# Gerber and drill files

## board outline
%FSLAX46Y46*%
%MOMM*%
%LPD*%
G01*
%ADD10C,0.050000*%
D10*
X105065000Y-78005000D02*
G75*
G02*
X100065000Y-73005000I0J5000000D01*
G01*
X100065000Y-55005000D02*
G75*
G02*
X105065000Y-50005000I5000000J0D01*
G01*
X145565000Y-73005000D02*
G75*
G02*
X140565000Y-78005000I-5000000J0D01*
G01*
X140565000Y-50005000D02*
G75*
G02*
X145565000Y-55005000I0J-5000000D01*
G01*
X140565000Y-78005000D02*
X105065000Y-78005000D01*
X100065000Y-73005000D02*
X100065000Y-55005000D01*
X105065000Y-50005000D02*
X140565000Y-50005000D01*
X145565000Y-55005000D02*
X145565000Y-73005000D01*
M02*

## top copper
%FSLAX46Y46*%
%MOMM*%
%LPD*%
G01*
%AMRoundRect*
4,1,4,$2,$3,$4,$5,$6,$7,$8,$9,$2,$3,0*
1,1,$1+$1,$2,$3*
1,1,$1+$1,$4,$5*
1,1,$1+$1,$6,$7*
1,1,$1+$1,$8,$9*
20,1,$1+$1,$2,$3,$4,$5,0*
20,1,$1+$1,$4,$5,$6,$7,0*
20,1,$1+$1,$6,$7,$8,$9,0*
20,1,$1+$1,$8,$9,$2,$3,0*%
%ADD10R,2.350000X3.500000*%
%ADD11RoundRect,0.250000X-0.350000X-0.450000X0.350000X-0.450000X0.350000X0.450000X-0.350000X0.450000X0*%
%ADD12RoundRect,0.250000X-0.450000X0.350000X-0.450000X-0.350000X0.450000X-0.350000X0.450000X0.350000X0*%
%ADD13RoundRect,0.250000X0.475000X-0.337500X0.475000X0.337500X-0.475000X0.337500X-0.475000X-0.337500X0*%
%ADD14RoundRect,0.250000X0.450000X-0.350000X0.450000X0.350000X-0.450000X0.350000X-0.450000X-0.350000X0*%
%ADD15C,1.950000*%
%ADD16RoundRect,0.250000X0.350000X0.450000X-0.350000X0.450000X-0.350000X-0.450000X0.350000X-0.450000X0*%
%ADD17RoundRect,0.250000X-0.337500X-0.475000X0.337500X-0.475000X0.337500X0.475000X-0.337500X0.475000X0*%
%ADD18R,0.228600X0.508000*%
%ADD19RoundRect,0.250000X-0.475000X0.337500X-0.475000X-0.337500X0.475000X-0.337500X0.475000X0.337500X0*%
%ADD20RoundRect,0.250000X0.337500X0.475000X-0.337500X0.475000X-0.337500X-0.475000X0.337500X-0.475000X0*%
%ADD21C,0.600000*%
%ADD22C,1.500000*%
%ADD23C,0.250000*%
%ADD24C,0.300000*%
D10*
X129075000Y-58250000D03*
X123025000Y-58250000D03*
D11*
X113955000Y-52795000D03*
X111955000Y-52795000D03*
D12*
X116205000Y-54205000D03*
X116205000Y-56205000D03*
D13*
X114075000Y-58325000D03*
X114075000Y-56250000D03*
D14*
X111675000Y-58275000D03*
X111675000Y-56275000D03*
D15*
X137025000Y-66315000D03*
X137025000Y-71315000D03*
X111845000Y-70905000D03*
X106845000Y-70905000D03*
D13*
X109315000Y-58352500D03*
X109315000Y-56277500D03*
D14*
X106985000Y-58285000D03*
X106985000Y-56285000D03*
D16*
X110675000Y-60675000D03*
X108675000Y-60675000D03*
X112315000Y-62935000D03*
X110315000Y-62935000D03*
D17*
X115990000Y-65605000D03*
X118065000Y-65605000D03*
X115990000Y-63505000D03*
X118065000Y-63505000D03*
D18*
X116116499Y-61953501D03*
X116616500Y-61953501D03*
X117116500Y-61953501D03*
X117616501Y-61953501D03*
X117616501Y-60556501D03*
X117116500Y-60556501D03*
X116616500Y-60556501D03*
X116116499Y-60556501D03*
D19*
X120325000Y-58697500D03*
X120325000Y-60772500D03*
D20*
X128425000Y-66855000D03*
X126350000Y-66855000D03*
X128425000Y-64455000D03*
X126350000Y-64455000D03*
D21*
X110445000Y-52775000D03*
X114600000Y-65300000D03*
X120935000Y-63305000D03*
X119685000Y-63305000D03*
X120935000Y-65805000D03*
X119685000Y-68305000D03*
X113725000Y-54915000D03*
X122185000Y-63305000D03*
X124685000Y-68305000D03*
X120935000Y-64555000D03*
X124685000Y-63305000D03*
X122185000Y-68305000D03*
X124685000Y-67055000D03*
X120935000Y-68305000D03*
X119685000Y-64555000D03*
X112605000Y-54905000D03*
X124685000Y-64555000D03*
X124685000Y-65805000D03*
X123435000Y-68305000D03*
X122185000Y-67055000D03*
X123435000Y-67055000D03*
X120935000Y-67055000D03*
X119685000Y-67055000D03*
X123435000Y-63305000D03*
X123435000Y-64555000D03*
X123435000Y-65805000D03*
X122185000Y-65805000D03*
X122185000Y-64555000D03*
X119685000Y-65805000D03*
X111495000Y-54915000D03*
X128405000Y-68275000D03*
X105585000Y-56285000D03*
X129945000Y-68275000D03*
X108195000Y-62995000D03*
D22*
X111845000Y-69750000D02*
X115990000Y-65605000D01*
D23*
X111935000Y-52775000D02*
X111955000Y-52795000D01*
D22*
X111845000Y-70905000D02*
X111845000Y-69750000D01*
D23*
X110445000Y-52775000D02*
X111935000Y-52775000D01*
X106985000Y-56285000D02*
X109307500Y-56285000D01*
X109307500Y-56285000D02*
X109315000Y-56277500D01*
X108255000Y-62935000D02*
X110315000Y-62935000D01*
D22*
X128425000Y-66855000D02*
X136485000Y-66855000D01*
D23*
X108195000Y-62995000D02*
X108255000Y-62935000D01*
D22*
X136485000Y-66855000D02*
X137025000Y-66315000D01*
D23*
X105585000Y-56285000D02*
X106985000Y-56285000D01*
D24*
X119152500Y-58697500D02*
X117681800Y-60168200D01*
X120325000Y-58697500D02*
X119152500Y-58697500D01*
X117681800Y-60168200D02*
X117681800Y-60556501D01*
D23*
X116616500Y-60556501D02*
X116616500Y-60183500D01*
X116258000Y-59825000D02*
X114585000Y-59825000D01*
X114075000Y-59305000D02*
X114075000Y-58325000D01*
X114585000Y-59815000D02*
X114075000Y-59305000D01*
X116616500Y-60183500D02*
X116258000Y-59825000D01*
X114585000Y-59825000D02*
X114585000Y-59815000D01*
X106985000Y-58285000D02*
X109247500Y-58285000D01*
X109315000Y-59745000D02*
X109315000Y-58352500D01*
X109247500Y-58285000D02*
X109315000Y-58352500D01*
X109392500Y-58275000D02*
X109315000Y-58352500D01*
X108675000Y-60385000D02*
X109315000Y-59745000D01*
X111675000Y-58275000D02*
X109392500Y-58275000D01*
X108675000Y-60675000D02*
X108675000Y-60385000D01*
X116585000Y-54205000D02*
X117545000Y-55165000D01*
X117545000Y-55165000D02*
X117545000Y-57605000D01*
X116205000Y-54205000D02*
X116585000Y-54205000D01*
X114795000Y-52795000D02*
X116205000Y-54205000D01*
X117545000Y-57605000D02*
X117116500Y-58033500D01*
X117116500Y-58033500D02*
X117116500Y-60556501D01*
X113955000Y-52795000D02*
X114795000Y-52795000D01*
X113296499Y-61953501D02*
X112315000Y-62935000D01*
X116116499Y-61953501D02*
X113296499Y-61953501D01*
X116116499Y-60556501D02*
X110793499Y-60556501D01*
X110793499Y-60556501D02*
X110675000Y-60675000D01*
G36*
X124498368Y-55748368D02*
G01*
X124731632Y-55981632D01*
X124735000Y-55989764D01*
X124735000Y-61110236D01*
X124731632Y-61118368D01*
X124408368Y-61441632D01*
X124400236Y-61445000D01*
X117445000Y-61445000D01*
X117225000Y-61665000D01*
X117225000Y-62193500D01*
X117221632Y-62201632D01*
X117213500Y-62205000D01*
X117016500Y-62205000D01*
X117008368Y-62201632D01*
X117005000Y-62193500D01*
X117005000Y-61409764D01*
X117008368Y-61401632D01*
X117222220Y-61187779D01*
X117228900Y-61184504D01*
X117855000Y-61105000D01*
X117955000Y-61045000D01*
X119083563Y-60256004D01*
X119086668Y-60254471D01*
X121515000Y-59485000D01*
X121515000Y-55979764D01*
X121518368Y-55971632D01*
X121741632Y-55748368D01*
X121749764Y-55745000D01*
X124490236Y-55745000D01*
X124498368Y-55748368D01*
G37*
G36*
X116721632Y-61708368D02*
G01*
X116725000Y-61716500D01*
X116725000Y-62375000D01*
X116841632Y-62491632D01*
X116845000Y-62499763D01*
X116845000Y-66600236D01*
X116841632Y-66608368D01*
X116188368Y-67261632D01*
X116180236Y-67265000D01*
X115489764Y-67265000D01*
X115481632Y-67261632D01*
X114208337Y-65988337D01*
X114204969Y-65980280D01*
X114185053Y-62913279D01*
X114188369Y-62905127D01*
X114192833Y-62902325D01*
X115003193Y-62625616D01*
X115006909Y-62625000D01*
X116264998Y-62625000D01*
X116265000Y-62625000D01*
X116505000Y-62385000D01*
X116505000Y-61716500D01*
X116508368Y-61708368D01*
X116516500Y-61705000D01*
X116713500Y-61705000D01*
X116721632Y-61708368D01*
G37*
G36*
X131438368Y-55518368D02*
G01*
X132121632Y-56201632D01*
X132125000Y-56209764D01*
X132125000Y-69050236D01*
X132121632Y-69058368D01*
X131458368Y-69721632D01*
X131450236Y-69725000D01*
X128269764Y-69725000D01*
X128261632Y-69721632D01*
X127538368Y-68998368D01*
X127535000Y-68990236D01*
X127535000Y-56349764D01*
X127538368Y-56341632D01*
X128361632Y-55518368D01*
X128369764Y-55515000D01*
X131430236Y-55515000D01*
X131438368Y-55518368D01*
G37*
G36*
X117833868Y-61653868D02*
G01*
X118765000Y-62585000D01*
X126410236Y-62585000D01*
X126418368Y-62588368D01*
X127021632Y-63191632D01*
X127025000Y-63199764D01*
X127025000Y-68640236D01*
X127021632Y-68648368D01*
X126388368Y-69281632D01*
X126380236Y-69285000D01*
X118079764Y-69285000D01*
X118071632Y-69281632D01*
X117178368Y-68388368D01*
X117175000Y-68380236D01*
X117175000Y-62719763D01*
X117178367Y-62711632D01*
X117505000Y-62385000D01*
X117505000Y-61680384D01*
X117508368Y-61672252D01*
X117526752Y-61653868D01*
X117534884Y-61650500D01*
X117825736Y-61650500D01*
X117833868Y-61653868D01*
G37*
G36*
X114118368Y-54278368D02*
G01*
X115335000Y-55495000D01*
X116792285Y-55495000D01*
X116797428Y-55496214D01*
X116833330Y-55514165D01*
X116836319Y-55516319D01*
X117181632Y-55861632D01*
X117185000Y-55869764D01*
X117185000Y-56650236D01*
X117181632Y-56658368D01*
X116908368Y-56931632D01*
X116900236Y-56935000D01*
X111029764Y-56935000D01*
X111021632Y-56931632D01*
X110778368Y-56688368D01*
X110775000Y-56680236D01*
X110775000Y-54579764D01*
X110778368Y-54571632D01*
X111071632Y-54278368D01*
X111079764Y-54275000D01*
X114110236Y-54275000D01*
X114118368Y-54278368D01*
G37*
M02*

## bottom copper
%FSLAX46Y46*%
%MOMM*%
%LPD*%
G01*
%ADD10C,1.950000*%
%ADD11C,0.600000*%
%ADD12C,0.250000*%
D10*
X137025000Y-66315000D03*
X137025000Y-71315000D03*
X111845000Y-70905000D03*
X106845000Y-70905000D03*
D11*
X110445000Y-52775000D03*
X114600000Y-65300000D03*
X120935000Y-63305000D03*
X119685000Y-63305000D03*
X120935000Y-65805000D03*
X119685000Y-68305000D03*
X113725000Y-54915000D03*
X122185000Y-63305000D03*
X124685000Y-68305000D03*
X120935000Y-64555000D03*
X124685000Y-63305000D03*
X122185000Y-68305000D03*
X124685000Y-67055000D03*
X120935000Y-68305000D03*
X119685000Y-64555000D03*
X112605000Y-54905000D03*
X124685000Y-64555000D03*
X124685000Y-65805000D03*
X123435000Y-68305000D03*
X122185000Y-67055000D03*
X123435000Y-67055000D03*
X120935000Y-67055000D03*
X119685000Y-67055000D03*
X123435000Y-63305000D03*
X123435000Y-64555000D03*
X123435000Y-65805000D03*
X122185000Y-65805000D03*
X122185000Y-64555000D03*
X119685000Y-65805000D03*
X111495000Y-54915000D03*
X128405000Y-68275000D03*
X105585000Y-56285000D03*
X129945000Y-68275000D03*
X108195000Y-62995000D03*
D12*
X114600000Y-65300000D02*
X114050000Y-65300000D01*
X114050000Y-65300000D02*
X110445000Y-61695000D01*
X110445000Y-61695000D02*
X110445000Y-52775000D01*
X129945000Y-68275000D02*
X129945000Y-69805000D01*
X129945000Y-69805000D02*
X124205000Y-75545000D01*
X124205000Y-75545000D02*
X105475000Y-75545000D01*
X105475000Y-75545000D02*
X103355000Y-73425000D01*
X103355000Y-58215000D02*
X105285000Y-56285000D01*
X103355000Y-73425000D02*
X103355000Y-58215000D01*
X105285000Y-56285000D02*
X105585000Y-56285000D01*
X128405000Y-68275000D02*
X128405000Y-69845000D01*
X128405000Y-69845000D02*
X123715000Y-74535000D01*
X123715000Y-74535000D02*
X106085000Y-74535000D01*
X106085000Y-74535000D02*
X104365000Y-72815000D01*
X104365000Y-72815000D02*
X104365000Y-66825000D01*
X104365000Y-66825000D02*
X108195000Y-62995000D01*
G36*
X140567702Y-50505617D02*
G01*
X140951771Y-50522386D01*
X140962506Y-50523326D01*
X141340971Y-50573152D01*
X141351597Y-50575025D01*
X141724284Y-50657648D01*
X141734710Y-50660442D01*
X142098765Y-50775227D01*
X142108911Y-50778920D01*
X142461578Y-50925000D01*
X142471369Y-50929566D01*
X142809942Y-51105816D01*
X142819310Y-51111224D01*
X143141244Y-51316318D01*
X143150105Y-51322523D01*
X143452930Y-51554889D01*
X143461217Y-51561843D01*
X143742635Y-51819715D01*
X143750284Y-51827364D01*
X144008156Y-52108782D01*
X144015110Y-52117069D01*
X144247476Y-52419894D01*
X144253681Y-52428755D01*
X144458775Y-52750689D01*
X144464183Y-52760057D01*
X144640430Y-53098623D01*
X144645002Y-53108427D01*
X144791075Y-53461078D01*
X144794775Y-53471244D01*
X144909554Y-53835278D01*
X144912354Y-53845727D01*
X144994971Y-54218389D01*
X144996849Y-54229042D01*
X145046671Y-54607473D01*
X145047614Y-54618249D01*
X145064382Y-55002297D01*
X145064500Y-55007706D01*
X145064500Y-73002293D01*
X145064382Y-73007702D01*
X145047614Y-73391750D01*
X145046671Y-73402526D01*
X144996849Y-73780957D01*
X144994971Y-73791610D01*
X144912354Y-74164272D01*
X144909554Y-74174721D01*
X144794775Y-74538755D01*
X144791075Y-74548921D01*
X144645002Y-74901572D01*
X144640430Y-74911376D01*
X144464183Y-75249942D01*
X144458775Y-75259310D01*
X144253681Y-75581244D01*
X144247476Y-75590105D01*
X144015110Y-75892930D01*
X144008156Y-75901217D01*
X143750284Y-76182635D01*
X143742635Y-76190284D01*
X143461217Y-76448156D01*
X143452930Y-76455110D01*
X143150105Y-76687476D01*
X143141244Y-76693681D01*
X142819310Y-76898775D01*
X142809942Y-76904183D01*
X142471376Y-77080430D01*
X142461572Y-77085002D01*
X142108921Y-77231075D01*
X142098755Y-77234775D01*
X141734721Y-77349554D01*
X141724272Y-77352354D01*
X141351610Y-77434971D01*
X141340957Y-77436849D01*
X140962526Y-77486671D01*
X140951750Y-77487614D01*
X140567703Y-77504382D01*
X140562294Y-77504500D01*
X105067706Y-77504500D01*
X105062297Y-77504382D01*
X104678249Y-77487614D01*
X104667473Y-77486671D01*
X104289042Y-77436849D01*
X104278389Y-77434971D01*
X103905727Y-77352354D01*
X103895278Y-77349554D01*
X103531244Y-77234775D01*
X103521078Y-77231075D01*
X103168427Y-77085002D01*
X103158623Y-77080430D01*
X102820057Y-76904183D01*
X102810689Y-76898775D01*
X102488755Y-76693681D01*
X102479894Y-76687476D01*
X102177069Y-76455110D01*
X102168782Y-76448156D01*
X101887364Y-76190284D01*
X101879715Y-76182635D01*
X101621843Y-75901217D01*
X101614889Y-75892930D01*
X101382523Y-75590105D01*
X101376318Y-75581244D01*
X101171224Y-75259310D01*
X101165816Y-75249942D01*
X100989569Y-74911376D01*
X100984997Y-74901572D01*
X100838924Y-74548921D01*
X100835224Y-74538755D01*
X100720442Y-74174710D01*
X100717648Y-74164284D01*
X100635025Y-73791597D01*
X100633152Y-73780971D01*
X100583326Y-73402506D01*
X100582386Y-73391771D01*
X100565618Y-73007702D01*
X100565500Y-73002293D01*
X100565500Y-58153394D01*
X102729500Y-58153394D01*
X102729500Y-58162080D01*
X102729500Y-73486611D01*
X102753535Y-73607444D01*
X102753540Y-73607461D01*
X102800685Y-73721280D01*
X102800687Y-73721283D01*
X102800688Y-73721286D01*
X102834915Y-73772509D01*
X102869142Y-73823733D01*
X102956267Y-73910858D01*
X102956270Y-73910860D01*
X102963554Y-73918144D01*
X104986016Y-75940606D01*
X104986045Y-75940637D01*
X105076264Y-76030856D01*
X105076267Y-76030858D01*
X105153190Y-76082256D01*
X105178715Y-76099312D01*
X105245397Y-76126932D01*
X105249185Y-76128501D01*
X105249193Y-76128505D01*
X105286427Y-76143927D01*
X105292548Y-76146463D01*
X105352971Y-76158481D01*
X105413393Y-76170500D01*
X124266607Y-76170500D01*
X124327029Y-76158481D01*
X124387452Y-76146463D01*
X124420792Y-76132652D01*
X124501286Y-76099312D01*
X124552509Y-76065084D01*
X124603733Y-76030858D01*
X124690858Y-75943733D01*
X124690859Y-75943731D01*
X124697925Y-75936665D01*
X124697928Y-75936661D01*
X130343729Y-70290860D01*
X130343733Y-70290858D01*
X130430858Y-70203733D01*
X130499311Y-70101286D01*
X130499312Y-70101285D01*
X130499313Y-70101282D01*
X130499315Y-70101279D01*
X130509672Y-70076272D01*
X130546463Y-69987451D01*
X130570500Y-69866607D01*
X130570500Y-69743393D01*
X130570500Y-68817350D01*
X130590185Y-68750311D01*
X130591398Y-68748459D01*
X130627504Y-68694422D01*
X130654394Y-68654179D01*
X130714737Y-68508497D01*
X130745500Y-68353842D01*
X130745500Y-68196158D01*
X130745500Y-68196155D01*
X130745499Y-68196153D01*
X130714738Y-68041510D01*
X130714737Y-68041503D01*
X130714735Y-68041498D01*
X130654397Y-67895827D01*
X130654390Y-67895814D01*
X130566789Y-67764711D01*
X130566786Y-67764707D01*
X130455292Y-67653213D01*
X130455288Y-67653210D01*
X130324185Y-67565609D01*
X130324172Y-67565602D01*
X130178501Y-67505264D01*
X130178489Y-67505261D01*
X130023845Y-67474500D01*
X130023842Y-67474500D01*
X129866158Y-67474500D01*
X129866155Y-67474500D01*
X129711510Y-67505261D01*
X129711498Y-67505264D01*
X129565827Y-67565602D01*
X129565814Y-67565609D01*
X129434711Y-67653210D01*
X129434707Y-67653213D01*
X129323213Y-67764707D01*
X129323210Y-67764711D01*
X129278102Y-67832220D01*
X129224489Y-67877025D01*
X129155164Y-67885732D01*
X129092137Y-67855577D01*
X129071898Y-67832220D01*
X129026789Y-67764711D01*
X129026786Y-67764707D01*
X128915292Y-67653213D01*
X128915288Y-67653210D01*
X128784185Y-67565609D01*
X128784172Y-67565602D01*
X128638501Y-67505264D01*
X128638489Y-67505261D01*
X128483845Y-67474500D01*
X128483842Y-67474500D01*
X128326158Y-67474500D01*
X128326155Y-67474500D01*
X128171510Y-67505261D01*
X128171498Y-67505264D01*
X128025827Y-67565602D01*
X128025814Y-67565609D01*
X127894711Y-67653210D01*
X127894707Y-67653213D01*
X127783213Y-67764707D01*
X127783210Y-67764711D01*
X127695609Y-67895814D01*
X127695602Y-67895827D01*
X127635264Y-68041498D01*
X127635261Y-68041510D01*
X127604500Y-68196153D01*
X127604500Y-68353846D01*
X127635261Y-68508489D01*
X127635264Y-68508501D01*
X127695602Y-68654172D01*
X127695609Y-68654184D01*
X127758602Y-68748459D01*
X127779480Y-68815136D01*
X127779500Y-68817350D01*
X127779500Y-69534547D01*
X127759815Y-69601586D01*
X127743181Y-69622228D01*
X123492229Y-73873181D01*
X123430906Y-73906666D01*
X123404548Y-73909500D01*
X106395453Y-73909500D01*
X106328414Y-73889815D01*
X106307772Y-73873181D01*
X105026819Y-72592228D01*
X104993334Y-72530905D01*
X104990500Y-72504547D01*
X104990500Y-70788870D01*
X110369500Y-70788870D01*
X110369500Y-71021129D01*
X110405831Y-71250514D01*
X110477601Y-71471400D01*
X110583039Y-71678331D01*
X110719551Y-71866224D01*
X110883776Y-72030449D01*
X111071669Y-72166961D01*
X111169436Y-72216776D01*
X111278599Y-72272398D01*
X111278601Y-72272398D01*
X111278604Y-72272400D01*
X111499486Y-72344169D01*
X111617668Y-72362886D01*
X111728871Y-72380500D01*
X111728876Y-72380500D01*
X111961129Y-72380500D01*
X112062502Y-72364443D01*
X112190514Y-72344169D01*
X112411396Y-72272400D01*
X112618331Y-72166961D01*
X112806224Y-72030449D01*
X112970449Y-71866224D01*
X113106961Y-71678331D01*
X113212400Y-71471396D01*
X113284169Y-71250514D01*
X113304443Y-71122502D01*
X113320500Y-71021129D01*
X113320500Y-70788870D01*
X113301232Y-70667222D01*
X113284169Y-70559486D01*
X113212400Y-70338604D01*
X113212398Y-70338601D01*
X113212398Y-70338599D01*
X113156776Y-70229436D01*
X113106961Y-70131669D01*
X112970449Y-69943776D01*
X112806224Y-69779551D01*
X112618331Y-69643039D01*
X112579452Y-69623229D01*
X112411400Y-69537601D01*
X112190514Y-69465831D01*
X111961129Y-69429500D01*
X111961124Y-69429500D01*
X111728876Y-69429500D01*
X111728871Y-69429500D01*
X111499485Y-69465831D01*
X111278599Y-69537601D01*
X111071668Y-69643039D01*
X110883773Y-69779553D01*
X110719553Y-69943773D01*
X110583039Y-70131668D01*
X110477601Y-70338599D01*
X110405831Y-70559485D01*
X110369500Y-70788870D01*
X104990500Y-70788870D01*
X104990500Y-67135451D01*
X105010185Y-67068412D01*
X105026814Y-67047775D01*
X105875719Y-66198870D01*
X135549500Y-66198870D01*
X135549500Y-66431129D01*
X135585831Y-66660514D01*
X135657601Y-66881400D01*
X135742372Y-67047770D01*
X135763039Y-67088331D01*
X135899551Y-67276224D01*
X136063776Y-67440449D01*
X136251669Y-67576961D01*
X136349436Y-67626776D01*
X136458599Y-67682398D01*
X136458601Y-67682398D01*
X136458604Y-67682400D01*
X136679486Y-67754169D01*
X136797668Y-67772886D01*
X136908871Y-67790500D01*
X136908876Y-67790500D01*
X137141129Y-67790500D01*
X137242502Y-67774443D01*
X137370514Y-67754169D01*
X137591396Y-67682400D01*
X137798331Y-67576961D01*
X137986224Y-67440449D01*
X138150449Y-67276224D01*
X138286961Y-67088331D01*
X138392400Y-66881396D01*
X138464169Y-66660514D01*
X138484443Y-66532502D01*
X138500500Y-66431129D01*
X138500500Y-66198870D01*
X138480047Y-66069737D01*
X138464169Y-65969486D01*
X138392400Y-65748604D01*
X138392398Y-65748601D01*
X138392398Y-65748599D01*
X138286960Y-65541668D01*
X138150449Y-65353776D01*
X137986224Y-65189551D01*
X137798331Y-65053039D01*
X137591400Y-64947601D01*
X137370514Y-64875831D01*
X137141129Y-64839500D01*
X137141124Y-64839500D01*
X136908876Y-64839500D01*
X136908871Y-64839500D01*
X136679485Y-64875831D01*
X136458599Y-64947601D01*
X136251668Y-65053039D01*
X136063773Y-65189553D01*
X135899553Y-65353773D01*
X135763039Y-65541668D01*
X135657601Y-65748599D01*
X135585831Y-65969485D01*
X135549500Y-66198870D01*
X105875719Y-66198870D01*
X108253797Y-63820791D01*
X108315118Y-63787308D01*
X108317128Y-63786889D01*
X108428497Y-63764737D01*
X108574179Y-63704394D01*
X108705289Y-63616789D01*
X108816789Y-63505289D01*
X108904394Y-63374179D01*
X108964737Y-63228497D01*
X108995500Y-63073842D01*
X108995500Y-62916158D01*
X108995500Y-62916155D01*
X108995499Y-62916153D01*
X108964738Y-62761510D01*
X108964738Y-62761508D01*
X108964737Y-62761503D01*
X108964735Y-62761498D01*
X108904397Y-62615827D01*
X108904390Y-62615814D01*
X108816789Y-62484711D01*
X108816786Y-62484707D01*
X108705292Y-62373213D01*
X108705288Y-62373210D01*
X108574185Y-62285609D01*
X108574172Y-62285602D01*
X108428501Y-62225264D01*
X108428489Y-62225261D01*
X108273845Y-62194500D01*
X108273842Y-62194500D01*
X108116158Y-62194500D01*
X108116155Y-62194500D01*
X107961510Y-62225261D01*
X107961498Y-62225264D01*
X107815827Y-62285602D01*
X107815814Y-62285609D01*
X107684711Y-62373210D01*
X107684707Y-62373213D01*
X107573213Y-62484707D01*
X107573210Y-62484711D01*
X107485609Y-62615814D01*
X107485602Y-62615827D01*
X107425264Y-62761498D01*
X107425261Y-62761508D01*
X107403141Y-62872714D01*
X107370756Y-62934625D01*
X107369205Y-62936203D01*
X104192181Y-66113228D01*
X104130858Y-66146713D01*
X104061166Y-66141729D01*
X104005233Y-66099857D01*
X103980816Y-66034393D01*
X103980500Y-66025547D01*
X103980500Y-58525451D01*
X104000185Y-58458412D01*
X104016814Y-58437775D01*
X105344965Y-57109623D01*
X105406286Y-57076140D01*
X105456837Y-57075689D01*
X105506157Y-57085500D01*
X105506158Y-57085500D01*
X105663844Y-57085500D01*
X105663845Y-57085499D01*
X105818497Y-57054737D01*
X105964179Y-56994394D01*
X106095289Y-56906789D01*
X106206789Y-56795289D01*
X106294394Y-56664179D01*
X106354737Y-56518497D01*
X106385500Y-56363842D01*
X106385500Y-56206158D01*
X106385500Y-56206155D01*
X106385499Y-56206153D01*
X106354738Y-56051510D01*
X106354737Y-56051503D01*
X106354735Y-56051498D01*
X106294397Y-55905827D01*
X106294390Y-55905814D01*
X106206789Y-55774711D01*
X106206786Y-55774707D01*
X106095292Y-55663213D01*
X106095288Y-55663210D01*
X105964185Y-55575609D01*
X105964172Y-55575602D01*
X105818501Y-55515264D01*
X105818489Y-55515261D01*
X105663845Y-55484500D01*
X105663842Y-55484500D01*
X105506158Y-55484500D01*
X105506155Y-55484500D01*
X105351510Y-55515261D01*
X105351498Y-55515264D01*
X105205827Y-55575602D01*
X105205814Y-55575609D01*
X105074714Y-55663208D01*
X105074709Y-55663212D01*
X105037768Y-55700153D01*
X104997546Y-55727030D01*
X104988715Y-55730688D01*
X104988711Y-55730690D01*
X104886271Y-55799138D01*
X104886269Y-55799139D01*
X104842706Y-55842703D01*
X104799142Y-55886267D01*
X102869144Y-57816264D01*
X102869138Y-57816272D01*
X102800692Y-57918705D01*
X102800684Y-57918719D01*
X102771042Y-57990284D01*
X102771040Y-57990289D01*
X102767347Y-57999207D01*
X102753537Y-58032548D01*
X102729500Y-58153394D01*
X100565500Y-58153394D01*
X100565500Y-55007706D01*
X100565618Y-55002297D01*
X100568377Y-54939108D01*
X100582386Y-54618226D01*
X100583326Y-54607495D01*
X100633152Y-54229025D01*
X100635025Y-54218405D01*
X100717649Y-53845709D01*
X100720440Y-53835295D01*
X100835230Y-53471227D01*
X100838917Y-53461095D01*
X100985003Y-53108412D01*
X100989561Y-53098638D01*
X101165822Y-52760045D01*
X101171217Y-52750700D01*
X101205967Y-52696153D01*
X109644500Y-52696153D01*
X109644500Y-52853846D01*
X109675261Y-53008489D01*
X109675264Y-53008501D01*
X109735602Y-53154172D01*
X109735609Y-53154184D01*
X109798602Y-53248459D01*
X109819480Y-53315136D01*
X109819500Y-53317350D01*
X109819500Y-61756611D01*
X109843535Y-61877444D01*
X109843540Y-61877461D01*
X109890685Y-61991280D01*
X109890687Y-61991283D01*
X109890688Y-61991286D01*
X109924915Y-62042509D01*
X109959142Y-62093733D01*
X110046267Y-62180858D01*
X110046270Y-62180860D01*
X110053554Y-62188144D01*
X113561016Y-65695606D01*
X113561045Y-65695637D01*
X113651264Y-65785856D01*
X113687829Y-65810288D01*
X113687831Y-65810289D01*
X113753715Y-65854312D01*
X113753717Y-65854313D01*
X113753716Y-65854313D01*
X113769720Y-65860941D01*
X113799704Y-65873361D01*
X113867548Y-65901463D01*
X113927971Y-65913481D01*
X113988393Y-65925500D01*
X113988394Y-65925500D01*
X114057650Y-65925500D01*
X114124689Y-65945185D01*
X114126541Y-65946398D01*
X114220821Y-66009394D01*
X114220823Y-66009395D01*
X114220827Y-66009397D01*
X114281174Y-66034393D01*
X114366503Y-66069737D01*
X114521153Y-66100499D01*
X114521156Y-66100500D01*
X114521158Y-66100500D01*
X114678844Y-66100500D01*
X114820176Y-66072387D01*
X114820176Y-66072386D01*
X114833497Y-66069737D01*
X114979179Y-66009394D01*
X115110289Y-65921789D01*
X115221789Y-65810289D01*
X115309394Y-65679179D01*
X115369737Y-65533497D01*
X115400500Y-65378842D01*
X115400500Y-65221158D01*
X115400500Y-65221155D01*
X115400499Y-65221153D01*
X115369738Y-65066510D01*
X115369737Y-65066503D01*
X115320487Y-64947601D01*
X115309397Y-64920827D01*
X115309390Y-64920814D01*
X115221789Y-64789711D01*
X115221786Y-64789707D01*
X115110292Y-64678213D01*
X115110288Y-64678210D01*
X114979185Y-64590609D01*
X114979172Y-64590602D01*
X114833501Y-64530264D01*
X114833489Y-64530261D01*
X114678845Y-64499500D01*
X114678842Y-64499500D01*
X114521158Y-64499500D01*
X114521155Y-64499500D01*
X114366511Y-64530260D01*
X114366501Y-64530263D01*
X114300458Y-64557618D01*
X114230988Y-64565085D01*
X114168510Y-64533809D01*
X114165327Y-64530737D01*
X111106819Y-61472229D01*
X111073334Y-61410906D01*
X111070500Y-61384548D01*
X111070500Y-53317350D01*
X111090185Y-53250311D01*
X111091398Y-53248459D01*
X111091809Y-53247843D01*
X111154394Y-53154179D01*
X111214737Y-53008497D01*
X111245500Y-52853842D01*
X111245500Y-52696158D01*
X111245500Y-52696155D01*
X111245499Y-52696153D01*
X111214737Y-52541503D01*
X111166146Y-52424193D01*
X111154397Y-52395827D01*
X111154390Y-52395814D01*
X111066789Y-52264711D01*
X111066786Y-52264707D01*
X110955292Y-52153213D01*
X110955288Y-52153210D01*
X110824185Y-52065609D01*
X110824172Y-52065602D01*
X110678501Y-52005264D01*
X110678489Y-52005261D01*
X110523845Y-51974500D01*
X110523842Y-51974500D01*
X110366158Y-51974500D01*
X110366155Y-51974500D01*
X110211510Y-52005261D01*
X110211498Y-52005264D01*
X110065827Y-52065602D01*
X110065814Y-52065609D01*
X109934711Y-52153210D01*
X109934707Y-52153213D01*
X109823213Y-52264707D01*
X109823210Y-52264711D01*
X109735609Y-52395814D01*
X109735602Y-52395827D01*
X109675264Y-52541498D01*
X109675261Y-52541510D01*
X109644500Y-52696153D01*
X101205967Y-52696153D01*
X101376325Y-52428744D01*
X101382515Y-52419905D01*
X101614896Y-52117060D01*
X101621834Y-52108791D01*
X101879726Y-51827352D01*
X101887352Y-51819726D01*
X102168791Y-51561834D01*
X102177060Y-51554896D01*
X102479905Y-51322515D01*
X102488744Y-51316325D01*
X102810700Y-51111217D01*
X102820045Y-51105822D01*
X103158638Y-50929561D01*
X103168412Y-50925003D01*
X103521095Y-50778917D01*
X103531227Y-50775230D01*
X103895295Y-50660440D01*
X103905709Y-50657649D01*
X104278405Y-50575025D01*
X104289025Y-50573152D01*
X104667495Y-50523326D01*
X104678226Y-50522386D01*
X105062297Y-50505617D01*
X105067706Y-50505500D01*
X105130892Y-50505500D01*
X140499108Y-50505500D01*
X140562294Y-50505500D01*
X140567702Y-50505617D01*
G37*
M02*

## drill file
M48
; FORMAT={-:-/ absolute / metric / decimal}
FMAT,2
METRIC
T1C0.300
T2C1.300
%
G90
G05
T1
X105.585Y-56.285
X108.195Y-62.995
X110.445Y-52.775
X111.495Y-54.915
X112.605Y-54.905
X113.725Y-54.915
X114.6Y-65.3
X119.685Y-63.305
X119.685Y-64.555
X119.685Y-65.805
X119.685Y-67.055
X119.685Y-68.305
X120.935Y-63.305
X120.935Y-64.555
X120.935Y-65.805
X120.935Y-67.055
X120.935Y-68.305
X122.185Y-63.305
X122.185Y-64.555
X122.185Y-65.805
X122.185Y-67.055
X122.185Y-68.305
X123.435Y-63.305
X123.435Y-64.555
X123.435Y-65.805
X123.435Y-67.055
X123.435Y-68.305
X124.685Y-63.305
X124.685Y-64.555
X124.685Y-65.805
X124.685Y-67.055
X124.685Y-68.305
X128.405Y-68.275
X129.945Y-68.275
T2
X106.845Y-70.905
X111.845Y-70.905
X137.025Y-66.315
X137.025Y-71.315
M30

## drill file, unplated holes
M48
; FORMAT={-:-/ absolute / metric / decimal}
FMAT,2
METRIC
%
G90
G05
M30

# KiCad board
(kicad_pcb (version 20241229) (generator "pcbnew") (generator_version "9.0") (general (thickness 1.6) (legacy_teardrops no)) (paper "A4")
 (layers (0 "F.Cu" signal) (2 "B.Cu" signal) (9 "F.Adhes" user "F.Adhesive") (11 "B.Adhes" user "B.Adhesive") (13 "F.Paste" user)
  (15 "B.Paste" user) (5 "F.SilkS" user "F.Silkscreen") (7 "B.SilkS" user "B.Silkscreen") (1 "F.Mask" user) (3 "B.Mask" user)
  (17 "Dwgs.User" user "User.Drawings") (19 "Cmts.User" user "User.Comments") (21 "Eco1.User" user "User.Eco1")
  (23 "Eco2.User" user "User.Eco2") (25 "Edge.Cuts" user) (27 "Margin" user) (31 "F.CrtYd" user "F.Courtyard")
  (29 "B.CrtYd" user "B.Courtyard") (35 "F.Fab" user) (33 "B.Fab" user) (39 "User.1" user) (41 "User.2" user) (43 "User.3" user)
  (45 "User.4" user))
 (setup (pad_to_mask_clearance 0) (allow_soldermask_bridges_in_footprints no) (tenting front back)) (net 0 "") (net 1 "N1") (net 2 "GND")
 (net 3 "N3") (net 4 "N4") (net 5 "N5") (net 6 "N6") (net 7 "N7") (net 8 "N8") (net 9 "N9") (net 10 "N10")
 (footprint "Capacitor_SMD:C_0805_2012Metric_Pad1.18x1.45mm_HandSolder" (layer "F.Cu") (at 127.3875 66.855 180)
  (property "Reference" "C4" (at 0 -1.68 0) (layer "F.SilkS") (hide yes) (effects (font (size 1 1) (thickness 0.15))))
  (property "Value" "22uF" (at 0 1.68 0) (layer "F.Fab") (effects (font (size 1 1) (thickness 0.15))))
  (pad "1" smd roundrect (at -1.0375 0 180) (size 1.175 1.45) (layers "F.Cu" "F.Mask" "F.Paste") (roundrect_rratio 0.212766) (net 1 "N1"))
  (pad "2" smd roundrect (at 1.0375 0 180) (size 1.175 1.45) (layers "F.Cu" "F.Mask" "F.Paste") (roundrect_rratio 0.212766) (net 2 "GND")))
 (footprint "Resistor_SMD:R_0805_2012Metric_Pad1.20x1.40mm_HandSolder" (layer "F.Cu") (at 111.315 62.935 180)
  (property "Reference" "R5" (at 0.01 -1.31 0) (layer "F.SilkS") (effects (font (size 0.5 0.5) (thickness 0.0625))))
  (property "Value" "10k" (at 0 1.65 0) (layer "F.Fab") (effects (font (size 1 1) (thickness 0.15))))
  (pad "1" smd roundrect (at -1 0 180) (size 1.2 1.4) (layers "F.Cu" "F.Mask" "F.Paste") (roundrect_rratio 0.208333) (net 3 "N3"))
  (pad "2" smd roundrect (at 1 0 180) (size 1.2 1.4) (layers "F.Cu" "F.Mask" "F.Paste") (roundrect_rratio 0.208333) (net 1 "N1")))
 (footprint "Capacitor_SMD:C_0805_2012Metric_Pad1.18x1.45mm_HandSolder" (layer "F.Cu") (at 114.075 57.2875 90)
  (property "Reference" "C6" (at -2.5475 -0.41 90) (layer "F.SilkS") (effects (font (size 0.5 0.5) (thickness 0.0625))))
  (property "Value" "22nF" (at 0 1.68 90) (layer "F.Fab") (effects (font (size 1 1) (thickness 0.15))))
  (pad "1" smd roundrect (at -1.0375 0 90) (size 1.175 1.45) (layers "F.Cu" "F.Mask" "F.Paste") (roundrect_rratio 0.212766) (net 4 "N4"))
  (pad "2" smd roundrect (at 1.0375 0 90) (size 1.175 1.45) (layers "F.Cu" "F.Mask" "F.Paste") (roundrect_rratio 0.212766) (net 2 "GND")))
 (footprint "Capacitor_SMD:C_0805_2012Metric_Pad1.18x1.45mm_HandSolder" (layer "F.Cu") (at 120.325 59.735 -90)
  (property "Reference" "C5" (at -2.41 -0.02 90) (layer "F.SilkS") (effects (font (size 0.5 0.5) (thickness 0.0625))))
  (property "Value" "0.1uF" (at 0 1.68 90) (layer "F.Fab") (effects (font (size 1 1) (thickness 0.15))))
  (pad "1" smd roundrect (at -1.0375 0 270) (size 1.175 1.45) (layers "F.Cu" "F.Mask" "F.Paste") (roundrect_rratio 0.212766) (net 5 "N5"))
  (pad "2" smd roundrect (at 1.0375 0 270) (size 1.175 1.45) (layers "F.Cu" "F.Mask" "F.Paste") (roundrect_rratio 0.212766) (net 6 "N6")))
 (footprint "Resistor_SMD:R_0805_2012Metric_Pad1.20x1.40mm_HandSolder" (layer "F.Cu") (at 112.955 52.795)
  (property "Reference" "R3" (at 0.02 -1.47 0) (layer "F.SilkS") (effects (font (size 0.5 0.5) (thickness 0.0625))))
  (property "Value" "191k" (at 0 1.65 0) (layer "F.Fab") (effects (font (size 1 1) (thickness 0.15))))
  (pad "1" smd roundrect (at -1 0) (size 1.2 1.4) (layers "F.Cu" "F.Mask" "F.Paste") (roundrect_rratio 0.208333) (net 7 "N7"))
  (pad "2" smd roundrect (at 1 0) (size 1.2 1.4) (layers "F.Cu" "F.Mask" "F.Paste") (roundrect_rratio 0.208333) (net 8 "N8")))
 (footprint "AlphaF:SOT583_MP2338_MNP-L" (layer "F.Cu") (at 116.8665 61.255001 90)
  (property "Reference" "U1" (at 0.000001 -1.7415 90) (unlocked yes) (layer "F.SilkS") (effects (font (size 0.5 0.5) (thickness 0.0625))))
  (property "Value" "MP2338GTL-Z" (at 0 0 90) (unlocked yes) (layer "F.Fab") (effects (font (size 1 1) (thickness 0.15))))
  (pad "1" smd rect (at -0.6985 -0.750001 90) (size 0.508 0.2286) (layers "F.Cu" "F.Mask" "F.Paste") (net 3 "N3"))
  (pad "2" smd rect (at -0.6985 -0.25 90) (size 0.508 0.2286) (layers "F.Cu" "F.Mask" "F.Paste") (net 7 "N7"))
  (pad "3" smd rect (at -0.6985 0.25 90) (size 0.508 0.2286) (layers "F.Cu" "F.Mask" "F.Paste") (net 6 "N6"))
  (pad "4" smd rect (at -0.6985 0.750001 90) (size 0.508 0.2286) (layers "F.Cu" "F.Mask" "F.Paste") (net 2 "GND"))
  (pad "5" smd rect (at 0.6985 0.750001 90) (size 0.508 0.2286) (layers "F.Cu" "F.Mask" "F.Paste") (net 5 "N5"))
  (pad "6" smd rect (at 0.6985 0.25 90) (size 0.508 0.2286) (layers "F.Cu" "F.Mask" "F.Paste") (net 8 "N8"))
  (pad "7" smd rect (at 0.6985 -0.25 90) (size 0.508 0.2286) (layers "F.Cu" "F.Mask" "F.Paste") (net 4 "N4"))
  (pad "8" smd rect (at 0.6985 -0.750001 90) (size 0.508 0.2286) (layers "F.Cu" "F.Mask" "F.Paste") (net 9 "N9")))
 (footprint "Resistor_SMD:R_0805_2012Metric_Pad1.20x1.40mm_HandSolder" (layer "F.Cu") (at 111.675 57.275 90)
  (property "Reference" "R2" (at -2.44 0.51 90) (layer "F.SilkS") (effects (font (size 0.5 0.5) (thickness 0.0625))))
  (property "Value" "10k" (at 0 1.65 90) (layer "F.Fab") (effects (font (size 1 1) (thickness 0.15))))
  (pad "1" smd roundrect (at -1 0 90) (size 1.2 1.4) (layers "F.Cu" "F.Mask" "F.Paste") (roundrect_rratio 0.208333) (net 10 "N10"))
  (pad "2" smd roundrect (at 1 0 90) (size 1.2 1.4) (layers "F.Cu" "F.Mask" "F.Paste") (roundrect_rratio 0.208333) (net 2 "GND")))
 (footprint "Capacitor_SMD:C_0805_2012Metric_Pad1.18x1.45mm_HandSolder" (layer "F.Cu") (at 117.0275 65.605)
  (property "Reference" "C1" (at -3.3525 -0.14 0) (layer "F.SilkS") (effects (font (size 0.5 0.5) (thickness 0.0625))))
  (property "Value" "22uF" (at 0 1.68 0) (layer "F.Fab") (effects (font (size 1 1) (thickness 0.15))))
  (pad "1" smd roundrect (at -1.0375 0) (size 1.175 1.45) (layers "F.Cu" "F.Mask" "F.Paste") (roundrect_rratio 0.212766) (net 7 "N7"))
  (pad "2" smd roundrect (at 1.0375 0) (size 1.175 1.45) (layers "F.Cu" "F.Mask" "F.Paste") (roundrect_rratio 0.212766) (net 2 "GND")))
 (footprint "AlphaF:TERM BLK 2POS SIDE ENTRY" (layer "F.Cu") (at 137.025 68.815 -90)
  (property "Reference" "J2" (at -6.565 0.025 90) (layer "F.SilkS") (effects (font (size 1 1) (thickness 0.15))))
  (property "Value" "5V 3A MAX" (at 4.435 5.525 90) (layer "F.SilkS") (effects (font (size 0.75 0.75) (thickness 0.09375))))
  (pad "1" thru_hole circle (at -2.5 0 270) (size 1.95 1.95) (drill 1.3) (layers "*.Cu" "*.Mask") (remove_unused_layers no) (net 1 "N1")
   (solder_mask_margin 0.102))
  (pad "2" thru_hole circle (at 2.5 0 270) (size 1.95 1.95) (drill 1.3) (layers "*.Cu" "*.Mask") (remove_unused_layers no) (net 2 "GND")
   (solder_mask_margin 0.102)))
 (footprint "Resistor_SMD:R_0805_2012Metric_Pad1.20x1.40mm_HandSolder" (layer "F.Cu") (at 116.205 55.205 -90)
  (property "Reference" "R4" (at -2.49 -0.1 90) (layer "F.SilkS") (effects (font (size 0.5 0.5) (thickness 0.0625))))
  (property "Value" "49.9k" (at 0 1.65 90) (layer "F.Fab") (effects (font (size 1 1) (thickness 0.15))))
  (pad "1" smd roundrect (at -1 0 270) (size 1.2 1.4) (layers "F.Cu" "F.Mask" "F.Paste") (roundrect_rratio 0.208333) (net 8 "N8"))
  (pad "2" smd roundrect (at 1 0 270) (size 1.2 1.4) (layers "F.Cu" "F.Mask" "F.Paste") (roundrect_rratio 0.208333) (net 2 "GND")))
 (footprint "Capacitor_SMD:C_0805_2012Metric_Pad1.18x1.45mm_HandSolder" (layer "F.Cu") (at 109.315 57.315 90)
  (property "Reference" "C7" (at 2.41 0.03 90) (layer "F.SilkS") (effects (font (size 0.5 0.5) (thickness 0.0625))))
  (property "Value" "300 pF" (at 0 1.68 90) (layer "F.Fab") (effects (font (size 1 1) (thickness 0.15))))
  (pad "1" smd roundrect (at -1.0375 0 90) (size 1.175 1.45) (layers "F.Cu" "F.Mask" "F.Paste") (roundrect_rratio 0.212766) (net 10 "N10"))
  (pad "2" smd roundrect (at 1.0375 0 90) (size 1.175 1.45) (layers "F.Cu" "F.Mask" "F.Paste") (roundrect_rratio 0.212766) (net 1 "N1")))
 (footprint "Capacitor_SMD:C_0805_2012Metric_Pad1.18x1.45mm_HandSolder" (layer "F.Cu") (at 117.0275 63.505)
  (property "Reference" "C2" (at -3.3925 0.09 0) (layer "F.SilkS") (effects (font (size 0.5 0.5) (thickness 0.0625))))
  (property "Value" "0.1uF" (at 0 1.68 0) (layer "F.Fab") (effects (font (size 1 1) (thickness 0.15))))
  (pad "1" smd roundrect (at -1.0375 0) (size 1.175 1.45) (layers "F.Cu" "F.Mask" "F.Paste") (roundrect_rratio 0.212766) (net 7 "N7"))
  (pad "2" smd roundrect (at 1.0375 0) (size 1.175 1.45) (layers "F.Cu" "F.Mask" "F.Paste") (roundrect_rratio 0.212766) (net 2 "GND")))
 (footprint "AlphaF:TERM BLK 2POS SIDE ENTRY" (layer "F.Cu") (at 109.345 70.905 180)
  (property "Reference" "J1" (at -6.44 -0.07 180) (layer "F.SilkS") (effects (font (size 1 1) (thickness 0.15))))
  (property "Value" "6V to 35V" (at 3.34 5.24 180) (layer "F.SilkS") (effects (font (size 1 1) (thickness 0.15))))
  (pad "1" thru_hole circle (at -2.5 0 180) (size 1.95 1.95) (drill 1.3) (layers "*.Cu" "*.Mask") (remove_unused_layers no) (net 7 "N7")
   (solder_mask_margin 0.102))
  (pad "2" thru_hole circle (at 2.5 0 180) (size 1.95 1.95) (drill 1.3) (layers "*.Cu" "*.Mask") (remove_unused_layers no) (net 2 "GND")
   (solder_mask_margin 0.102)))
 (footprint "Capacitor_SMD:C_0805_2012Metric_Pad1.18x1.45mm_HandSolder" (layer "F.Cu") (at 127.3875 64.455 180)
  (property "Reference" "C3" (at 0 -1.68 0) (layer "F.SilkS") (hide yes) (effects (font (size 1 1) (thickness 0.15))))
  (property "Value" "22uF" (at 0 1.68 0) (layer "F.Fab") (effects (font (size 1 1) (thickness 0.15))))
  (pad "1" smd roundrect (at -1.0375 0 180) (size 1.175 1.45) (layers "F.Cu" "F.Mask" "F.Paste") (roundrect_rratio 0.212766) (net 1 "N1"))
  (pad "2" smd roundrect (at 1.0375 0 180) (size 1.175 1.45) (layers "F.Cu" "F.Mask" "F.Paste") (roundrect_rratio 0.212766) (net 2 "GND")))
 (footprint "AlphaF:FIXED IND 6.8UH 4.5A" (layer "F.Cu") (at 126.05 58.25)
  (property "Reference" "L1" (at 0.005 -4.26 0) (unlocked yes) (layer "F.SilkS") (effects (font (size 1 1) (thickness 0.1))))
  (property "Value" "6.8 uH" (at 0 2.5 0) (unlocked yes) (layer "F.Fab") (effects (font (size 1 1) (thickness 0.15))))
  (pad "1" smd rect (at -3.025 0) (size 2.35 3.5) (layers "F.Cu" "F.Mask" "F.Paste") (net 6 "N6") (thermal_bridge_angle 45))
  (pad "2" smd rect (at 3.025 0) (size 2.35 3.5) (layers "F.Cu" "F.Mask" "F.Paste") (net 1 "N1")))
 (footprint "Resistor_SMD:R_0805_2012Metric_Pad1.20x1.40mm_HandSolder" (layer "F.Cu") (at 106.985 57.285 90)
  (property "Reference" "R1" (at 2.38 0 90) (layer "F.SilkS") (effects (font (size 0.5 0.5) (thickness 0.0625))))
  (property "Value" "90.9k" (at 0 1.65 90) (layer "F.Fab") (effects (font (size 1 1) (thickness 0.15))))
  (pad "1" smd roundrect (at -1 0 90) (size 1.2 1.4) (layers "F.Cu" "F.Mask" "F.Paste") (roundrect_rratio 0.208333) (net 10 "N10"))
  (pad "2" smd roundrect (at 1 0 90) (size 1.2 1.4) (layers "F.Cu" "F.Mask" "F.Paste") (roundrect_rratio 0.208333) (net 1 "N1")))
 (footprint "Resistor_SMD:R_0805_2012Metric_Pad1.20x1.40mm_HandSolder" (layer "F.Cu") (at 109.675 60.675 180)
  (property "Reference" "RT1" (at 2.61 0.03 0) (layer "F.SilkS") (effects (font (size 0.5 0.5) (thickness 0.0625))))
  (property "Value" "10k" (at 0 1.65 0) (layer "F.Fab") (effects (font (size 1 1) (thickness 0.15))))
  (pad "1" smd roundrect (at -1 0 180) (size 1.2 1.4) (layers "F.Cu" "F.Mask" "F.Paste") (roundrect_rratio 0.208333) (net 9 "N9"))
  (pad "2" smd roundrect (at 1 0 180) (size 1.2 1.4) (layers "F.Cu" "F.Mask" "F.Paste") (roundrect_rratio 0.208333) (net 10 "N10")))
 (gr_line (start 145.565 55.005) (end 145.565 73.005) (stroke (width 0.05) (type default)) (layer "Edge.Cuts"))
 (gr_arc (start 105.065 78.005) (mid 101.529466 76.540534) (end 100.065 73.005) (stroke (width 0.05) (type default)) (layer "Edge.Cuts"))
 (gr_arc (start 100.065 55.005) (mid 101.529466 51.469466) (end 105.065 50.005) (stroke (width 0.05) (type default)) (layer "Edge.Cuts"))
 (gr_line (start 100.065 73.005) (end 100.065 55.005) (stroke (width 0.05) (type default)) (layer "Edge.Cuts"))
 (gr_line (start 105.065 50.005) (end 140.565 50.005) (stroke (width 0.05) (type default)) (layer "Edge.Cuts"))
 (gr_arc (start 140.565 50.005) (mid 144.100534 51.469466) (end 145.565 55.005) (stroke (width 0.05) (type default)) (layer "Edge.Cuts"))
 (gr_line (start 140.565 78.005) (end 105.065 78.005) (stroke (width 0.05) (type default)) (layer "Edge.Cuts"))
 (gr_arc (start 145.565 73.005) (mid 144.100534 76.540534) (end 140.565 78.005) (stroke (width 0.05) (type default)) (layer "Edge.Cuts"))
 (segment (start 111.845 69.75) (end 115.99 65.605) (width 1.5) (layer "F.Cu") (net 7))
 (segment (start 111.935 52.775) (end 111.955 52.795) (width 0.25) (layer "F.Cu") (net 7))
 (segment (start 111.845 70.905) (end 111.845 69.75) (width 1.5) (layer "F.Cu") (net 7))
 (segment (start 110.445 52.775) (end 111.935 52.775) (width 0.25) (layer "F.Cu") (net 7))
 (via (at 110.445 52.775) (size 0.6) (drill 0.3) (layers "F.Cu" "B.Cu") (free yes) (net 7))
 (via (at 114.6 65.3) (size 0.6) (drill 0.3) (layers "F.Cu" "B.Cu") (free yes) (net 7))
 (segment (start 114.6 65.3) (end 114.05 65.3) (width 0.25) (layer "B.Cu") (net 7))
 (segment (start 114.05 65.3) (end 110.445 61.695) (width 0.25) (layer "B.Cu") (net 7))
 (segment (start 110.445 61.695) (end 110.445 52.775) (width 0.25) (layer "B.Cu") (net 7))
 (via (at 120.935 63.305) (size 0.6) (drill 0.3) (layers "F.Cu" "B.Cu") (free yes) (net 2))
 (via (at 119.685 63.305) (size 0.6) (drill 0.3) (layers "F.Cu" "B.Cu") (free yes) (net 2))
 (via (at 120.935 65.805) (size 0.6) (drill 0.3) (layers "F.Cu" "B.Cu") (free yes) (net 2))
 (via (at 119.685 68.305) (size 0.6) (drill 0.3) (layers "F.Cu" "B.Cu") (free yes) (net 2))
 (via (at 113.725 54.915) (size 0.6) (drill 0.3) (layers "F.Cu" "B.Cu") (free yes) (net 2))
 (via (at 122.185 63.305) (size 0.6) (drill 0.3) (layers "F.Cu" "B.Cu") (free yes) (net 2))
 (via (at 124.685 68.305) (size 0.6) (drill 0.3) (layers "F.Cu" "B.Cu") (free yes) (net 2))
 (via (at 120.935 64.555) (size 0.6) (drill 0.3) (layers "F.Cu" "B.Cu") (free yes) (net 2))
 (via (at 124.685 63.305) (size 0.6) (drill 0.3) (layers "F.Cu" "B.Cu") (free yes) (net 2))
 (via (at 122.185 68.305) (size 0.6) (drill 0.3) (layers "F.Cu" "B.Cu") (free yes) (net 2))
 (via (at 124.685 67.055) (size 0.6) (drill 0.3) (layers "F.Cu" "B.Cu") (free yes) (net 2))
 (via (at 120.935 68.305) (size 0.6) (drill 0.3) (layers "F.Cu" "B.Cu") (free yes) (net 2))
 (via (at 119.685 64.555) (size 0.6) (drill 0.3) (layers "F.Cu" "B.Cu") (free yes) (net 2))
 (via (at 112.605 54.905) (size 0.6) (drill 0.3) (layers "F.Cu" "B.Cu") (free yes) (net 2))
 (via (at 124.685 64.555) (size 0.6) (drill 0.3) (layers "F.Cu" "B.Cu") (free yes) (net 2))
 (via (at 124.685 65.805) (size 0.6) (drill 0.3) (layers "F.Cu" "B.Cu") (free yes) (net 2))
 (via (at 123.435 68.305) (size 0.6) (drill 0.3) (layers "F.Cu" "B.Cu") (free yes) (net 2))
 (via (at 122.185 67.055) (size 0.6) (drill 0.3) (layers "F.Cu" "B.Cu") (free yes) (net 2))
 (via (at 123.435 67.055) (size 0.6) (drill 0.3) (layers "F.Cu" "B.Cu") (free yes) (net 2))
 (via (at 120.935 67.055) (size 0.6) (drill 0.3) (layers "F.Cu" "B.Cu") (free yes) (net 2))
 (via (at 119.685 67.055) (size 0.6) (drill 0.3) (layers "F.Cu" "B.Cu") (free yes) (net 2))
 (via (at 123.435 63.305) (size 0.6) (drill 0.3) (layers "F.Cu" "B.Cu") (free yes) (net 2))
 (via (at 123.435 64.555) (size 0.6) (drill 0.3) (layers "F.Cu" "B.Cu") (free yes) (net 2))
 (via (at 123.435 65.805) (size 0.6) (drill 0.3) (layers "F.Cu" "B.Cu") (free yes) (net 2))
 (via (at 122.185 65.805) (size 0.6) (drill 0.3) (layers "F.Cu" "B.Cu") (free yes) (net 2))
 (via (at 122.185 64.555) (size 0.6) (drill 0.3) (layers "F.Cu" "B.Cu") (free yes) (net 2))
 (via (at 119.685 65.805) (size 0.6) (drill 0.3) (layers "F.Cu" "B.Cu") (free yes) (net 2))
 (via (at 111.495 54.915) (size 0.6) (drill 0.3) (layers "F.Cu" "B.Cu") (free yes) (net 2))
 (segment (start 106.985 56.285) (end 109.3075 56.285) (width 0.25) (layer "F.Cu") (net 1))
 (segment (start 109.3075 56.285) (end 109.315 56.2775) (width 0.25) (layer "F.Cu") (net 1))
 (segment (start 108.255 62.935) (end 110.315 62.935) (width 0.25) (layer "F.Cu") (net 1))
 (segment (start 128.425 66.855) (end 136.485 66.855) (width 1.5) (layer "F.Cu") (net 1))
 (segment (start 108.195 62.995) (end 108.255 62.935) (width 0.25) (layer "F.Cu") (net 1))
 (segment (start 136.485 66.855) (end 137.025 66.315) (width 1.5) (layer "F.Cu") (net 1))
 (segment (start 105.585 56.285) (end 106.985 56.285) (width 0.25) (layer "F.Cu") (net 1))
 (via (at 128.405 68.275) (size 0.6) (drill 0.3) (layers "F.Cu" "B.Cu") (free yes) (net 1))
 (via (at 105.585 56.285) (size 0.6) (drill 0.3) (layers "F.Cu" "B.Cu") (free yes) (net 1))
 (via (at 129.945 68.275) (size 0.6) (drill 0.3) (layers "F.Cu" "B.Cu") (free yes) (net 1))
 (via (at 108.195 62.995) (size 0.6) (drill 0.3) (layers "F.Cu" "B.Cu") (free yes) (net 1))
 (segment (start 124.205 75.545) (end 105.475 75.545) (width 0.25) (layer "B.Cu") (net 1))
 (segment (start 104.365 66.825) (end 108.195 62.995) (width 0.25) (layer "B.Cu") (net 1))
 (segment (start 129.945 69.805) (end 124.205 75.545) (width 0.25) (layer "B.Cu") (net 1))
 (segment (start 104.365 72.815) (end 104.365 66.825) (width 0.25) (layer "B.Cu") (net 1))
 (segment (start 123.715 74.535) (end 106.085 74.535) (width 0.25) (layer "B.Cu") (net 1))
 (segment (start 129.945 68.275) (end 129.945 69.805) (width 0.25) (layer "B.Cu") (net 1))
 (segment (start 128.405 68.275) (end 128.405 69.845) (width 0.25) (layer "B.Cu") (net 1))
 (segment (start 105.475 75.545) (end 103.355 73.425) (width 0.25) (layer "B.Cu") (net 1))
 (segment (start 106.085 74.535) (end 104.365 72.815) (width 0.25) (layer "B.Cu") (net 1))
 (segment (start 103.355 73.425) (end 103.355 58.215) (width 0.25) (layer "B.Cu") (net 1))
 (segment (start 105.285 56.285) (end 105.585 56.285) (width 0.25) (layer "B.Cu") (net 1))
 (segment (start 103.355 58.215) (end 105.285 56.285) (width 0.25) (layer "B.Cu") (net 1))
 (segment (start 128.405 69.845) (end 123.715 74.535) (width 0.25) (layer "B.Cu") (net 1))
 (segment (start 119.1525 58.6975) (end 117.6818 60.1682) (width 0.3) (layer "F.Cu") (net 5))
 (segment (start 120.325 58.6975) (end 119.1525 58.6975) (width 0.3) (layer "F.Cu") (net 5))
 (segment (start 117.6818 60.1682) (end 117.6818 60.556501) (width 0.3) (layer "F.Cu") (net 5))
 (segment (start 116.6165 60.556501) (end 116.6165 60.1835) (width 0.25) (layer "F.Cu") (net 4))
 (segment (start 116.258 59.825) (end 114.585 59.825) (width 0.25) (layer "F.Cu") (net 4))
 (segment (start 114.075 59.305) (end 114.075 58.325) (width 0.25) (layer "F.Cu") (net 4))
 (segment (start 114.585 59.815) (end 114.075 59.305) (width 0.25) (layer "F.Cu") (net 4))
 (segment (start 116.6165 60.1835) (end 116.258 59.825) (width 0.25) (layer "F.Cu") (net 4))
 (segment (start 114.585 59.825) (end 114.585 59.815) (width 0.25) (layer "F.Cu") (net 4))
 (segment (start 106.985 58.285) (end 109.2475 58.285) (width 0.25) (layer "F.Cu") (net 10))
 (segment (start 109.315 59.745) (end 109.315 58.3525) (width 0.25) (layer "F.Cu") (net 10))
 (segment (start 109.2475 58.285) (end 109.315 58.3525) (width 0.25) (layer "F.Cu") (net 10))
 (segment (start 109.3925 58.275) (end 109.315 58.3525) (width 0.25) (layer "F.Cu") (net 10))
 (segment (start 108.675 60.385) (end 109.315 59.745) (width 0.25) (layer "F.Cu") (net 10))
 (segment (start 111.675 58.275) (end 109.3925 58.275) (width 0.25) (layer "F.Cu") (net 10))
 (segment (start 108.675 60.675) (end 108.675 60.385) (width 0.25) (layer "F.Cu") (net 10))
 (segment (start 116.585 54.205) (end 117.545 55.165) (width 0.25) (layer "F.Cu") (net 8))
 (segment (start 117.545 55.165) (end 117.545 57.605) (width 0.25) (layer "F.Cu") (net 8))
 (segment (start 116.205 54.205) (end 116.585 54.205) (width 0.25) (layer "F.Cu") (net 8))
 (segment (start 114.795 52.795) (end 116.205 54.205) (width 0.25) (layer "F.Cu") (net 8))
 (segment (start 117.545 57.605) (end 117.1165 58.0335) (width 0.25) (layer "F.Cu") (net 8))
 (segment (start 117.1165 58.0335) (end 117.1165 60.556501) (width 0.25) (layer "F.Cu") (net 8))
 (segment (start 113.955 52.795) (end 114.795 52.795) (width 0.25) (layer "F.Cu") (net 8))
 (segment (start 113.296499 61.953501) (end 112.315 62.935) (width 0.25) (layer "F.Cu") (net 3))
 (segment (start 116.116499 61.953501) (end 113.296499 61.953501) (width 0.25) (layer "F.Cu") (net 3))
 (segment (start 116.116499 60.556501) (end 110.793499 60.556501) (width 0.25) (layer "F.Cu") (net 9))
 (segment (start 110.793499 60.556501) (end 110.675 60.675) (width 0.25) (layer "F.Cu") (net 9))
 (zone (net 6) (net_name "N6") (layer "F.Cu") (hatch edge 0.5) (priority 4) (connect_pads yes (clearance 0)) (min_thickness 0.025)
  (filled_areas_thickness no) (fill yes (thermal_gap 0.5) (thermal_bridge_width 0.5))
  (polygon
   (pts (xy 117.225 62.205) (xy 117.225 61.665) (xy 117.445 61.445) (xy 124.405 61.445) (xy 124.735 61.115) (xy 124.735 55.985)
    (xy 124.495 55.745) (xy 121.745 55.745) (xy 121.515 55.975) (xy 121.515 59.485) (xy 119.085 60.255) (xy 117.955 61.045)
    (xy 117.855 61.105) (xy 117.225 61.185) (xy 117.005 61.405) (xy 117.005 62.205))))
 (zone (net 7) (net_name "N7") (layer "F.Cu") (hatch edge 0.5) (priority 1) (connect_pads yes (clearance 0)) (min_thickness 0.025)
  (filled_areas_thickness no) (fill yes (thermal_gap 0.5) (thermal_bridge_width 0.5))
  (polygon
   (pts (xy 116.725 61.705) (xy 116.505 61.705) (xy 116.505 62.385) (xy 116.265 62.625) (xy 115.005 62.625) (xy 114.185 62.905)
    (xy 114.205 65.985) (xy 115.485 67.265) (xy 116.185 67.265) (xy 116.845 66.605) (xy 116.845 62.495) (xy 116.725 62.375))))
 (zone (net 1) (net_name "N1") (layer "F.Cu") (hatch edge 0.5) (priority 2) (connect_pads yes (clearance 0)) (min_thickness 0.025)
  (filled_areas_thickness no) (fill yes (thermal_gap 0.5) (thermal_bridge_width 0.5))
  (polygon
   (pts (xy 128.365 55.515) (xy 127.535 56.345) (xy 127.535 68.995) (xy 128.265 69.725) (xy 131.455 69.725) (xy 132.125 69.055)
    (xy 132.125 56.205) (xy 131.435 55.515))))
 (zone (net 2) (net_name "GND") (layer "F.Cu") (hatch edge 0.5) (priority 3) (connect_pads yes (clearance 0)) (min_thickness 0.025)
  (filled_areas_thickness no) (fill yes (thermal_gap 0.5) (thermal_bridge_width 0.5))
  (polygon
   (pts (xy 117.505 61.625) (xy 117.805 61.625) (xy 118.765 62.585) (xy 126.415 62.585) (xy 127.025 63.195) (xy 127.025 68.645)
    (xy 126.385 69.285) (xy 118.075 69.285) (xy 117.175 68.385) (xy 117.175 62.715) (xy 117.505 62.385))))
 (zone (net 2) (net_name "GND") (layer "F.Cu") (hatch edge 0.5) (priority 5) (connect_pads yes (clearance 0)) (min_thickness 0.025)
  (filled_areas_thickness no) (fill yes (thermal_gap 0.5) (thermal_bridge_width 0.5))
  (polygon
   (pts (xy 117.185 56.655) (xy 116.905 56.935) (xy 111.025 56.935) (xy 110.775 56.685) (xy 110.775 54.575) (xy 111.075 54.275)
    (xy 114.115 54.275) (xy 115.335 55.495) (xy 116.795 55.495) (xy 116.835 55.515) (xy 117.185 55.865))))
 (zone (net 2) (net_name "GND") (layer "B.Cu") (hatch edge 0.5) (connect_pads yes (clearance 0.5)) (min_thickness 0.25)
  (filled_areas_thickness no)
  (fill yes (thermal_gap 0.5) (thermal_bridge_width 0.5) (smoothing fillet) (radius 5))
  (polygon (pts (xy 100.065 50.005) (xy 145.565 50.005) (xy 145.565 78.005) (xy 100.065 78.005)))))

